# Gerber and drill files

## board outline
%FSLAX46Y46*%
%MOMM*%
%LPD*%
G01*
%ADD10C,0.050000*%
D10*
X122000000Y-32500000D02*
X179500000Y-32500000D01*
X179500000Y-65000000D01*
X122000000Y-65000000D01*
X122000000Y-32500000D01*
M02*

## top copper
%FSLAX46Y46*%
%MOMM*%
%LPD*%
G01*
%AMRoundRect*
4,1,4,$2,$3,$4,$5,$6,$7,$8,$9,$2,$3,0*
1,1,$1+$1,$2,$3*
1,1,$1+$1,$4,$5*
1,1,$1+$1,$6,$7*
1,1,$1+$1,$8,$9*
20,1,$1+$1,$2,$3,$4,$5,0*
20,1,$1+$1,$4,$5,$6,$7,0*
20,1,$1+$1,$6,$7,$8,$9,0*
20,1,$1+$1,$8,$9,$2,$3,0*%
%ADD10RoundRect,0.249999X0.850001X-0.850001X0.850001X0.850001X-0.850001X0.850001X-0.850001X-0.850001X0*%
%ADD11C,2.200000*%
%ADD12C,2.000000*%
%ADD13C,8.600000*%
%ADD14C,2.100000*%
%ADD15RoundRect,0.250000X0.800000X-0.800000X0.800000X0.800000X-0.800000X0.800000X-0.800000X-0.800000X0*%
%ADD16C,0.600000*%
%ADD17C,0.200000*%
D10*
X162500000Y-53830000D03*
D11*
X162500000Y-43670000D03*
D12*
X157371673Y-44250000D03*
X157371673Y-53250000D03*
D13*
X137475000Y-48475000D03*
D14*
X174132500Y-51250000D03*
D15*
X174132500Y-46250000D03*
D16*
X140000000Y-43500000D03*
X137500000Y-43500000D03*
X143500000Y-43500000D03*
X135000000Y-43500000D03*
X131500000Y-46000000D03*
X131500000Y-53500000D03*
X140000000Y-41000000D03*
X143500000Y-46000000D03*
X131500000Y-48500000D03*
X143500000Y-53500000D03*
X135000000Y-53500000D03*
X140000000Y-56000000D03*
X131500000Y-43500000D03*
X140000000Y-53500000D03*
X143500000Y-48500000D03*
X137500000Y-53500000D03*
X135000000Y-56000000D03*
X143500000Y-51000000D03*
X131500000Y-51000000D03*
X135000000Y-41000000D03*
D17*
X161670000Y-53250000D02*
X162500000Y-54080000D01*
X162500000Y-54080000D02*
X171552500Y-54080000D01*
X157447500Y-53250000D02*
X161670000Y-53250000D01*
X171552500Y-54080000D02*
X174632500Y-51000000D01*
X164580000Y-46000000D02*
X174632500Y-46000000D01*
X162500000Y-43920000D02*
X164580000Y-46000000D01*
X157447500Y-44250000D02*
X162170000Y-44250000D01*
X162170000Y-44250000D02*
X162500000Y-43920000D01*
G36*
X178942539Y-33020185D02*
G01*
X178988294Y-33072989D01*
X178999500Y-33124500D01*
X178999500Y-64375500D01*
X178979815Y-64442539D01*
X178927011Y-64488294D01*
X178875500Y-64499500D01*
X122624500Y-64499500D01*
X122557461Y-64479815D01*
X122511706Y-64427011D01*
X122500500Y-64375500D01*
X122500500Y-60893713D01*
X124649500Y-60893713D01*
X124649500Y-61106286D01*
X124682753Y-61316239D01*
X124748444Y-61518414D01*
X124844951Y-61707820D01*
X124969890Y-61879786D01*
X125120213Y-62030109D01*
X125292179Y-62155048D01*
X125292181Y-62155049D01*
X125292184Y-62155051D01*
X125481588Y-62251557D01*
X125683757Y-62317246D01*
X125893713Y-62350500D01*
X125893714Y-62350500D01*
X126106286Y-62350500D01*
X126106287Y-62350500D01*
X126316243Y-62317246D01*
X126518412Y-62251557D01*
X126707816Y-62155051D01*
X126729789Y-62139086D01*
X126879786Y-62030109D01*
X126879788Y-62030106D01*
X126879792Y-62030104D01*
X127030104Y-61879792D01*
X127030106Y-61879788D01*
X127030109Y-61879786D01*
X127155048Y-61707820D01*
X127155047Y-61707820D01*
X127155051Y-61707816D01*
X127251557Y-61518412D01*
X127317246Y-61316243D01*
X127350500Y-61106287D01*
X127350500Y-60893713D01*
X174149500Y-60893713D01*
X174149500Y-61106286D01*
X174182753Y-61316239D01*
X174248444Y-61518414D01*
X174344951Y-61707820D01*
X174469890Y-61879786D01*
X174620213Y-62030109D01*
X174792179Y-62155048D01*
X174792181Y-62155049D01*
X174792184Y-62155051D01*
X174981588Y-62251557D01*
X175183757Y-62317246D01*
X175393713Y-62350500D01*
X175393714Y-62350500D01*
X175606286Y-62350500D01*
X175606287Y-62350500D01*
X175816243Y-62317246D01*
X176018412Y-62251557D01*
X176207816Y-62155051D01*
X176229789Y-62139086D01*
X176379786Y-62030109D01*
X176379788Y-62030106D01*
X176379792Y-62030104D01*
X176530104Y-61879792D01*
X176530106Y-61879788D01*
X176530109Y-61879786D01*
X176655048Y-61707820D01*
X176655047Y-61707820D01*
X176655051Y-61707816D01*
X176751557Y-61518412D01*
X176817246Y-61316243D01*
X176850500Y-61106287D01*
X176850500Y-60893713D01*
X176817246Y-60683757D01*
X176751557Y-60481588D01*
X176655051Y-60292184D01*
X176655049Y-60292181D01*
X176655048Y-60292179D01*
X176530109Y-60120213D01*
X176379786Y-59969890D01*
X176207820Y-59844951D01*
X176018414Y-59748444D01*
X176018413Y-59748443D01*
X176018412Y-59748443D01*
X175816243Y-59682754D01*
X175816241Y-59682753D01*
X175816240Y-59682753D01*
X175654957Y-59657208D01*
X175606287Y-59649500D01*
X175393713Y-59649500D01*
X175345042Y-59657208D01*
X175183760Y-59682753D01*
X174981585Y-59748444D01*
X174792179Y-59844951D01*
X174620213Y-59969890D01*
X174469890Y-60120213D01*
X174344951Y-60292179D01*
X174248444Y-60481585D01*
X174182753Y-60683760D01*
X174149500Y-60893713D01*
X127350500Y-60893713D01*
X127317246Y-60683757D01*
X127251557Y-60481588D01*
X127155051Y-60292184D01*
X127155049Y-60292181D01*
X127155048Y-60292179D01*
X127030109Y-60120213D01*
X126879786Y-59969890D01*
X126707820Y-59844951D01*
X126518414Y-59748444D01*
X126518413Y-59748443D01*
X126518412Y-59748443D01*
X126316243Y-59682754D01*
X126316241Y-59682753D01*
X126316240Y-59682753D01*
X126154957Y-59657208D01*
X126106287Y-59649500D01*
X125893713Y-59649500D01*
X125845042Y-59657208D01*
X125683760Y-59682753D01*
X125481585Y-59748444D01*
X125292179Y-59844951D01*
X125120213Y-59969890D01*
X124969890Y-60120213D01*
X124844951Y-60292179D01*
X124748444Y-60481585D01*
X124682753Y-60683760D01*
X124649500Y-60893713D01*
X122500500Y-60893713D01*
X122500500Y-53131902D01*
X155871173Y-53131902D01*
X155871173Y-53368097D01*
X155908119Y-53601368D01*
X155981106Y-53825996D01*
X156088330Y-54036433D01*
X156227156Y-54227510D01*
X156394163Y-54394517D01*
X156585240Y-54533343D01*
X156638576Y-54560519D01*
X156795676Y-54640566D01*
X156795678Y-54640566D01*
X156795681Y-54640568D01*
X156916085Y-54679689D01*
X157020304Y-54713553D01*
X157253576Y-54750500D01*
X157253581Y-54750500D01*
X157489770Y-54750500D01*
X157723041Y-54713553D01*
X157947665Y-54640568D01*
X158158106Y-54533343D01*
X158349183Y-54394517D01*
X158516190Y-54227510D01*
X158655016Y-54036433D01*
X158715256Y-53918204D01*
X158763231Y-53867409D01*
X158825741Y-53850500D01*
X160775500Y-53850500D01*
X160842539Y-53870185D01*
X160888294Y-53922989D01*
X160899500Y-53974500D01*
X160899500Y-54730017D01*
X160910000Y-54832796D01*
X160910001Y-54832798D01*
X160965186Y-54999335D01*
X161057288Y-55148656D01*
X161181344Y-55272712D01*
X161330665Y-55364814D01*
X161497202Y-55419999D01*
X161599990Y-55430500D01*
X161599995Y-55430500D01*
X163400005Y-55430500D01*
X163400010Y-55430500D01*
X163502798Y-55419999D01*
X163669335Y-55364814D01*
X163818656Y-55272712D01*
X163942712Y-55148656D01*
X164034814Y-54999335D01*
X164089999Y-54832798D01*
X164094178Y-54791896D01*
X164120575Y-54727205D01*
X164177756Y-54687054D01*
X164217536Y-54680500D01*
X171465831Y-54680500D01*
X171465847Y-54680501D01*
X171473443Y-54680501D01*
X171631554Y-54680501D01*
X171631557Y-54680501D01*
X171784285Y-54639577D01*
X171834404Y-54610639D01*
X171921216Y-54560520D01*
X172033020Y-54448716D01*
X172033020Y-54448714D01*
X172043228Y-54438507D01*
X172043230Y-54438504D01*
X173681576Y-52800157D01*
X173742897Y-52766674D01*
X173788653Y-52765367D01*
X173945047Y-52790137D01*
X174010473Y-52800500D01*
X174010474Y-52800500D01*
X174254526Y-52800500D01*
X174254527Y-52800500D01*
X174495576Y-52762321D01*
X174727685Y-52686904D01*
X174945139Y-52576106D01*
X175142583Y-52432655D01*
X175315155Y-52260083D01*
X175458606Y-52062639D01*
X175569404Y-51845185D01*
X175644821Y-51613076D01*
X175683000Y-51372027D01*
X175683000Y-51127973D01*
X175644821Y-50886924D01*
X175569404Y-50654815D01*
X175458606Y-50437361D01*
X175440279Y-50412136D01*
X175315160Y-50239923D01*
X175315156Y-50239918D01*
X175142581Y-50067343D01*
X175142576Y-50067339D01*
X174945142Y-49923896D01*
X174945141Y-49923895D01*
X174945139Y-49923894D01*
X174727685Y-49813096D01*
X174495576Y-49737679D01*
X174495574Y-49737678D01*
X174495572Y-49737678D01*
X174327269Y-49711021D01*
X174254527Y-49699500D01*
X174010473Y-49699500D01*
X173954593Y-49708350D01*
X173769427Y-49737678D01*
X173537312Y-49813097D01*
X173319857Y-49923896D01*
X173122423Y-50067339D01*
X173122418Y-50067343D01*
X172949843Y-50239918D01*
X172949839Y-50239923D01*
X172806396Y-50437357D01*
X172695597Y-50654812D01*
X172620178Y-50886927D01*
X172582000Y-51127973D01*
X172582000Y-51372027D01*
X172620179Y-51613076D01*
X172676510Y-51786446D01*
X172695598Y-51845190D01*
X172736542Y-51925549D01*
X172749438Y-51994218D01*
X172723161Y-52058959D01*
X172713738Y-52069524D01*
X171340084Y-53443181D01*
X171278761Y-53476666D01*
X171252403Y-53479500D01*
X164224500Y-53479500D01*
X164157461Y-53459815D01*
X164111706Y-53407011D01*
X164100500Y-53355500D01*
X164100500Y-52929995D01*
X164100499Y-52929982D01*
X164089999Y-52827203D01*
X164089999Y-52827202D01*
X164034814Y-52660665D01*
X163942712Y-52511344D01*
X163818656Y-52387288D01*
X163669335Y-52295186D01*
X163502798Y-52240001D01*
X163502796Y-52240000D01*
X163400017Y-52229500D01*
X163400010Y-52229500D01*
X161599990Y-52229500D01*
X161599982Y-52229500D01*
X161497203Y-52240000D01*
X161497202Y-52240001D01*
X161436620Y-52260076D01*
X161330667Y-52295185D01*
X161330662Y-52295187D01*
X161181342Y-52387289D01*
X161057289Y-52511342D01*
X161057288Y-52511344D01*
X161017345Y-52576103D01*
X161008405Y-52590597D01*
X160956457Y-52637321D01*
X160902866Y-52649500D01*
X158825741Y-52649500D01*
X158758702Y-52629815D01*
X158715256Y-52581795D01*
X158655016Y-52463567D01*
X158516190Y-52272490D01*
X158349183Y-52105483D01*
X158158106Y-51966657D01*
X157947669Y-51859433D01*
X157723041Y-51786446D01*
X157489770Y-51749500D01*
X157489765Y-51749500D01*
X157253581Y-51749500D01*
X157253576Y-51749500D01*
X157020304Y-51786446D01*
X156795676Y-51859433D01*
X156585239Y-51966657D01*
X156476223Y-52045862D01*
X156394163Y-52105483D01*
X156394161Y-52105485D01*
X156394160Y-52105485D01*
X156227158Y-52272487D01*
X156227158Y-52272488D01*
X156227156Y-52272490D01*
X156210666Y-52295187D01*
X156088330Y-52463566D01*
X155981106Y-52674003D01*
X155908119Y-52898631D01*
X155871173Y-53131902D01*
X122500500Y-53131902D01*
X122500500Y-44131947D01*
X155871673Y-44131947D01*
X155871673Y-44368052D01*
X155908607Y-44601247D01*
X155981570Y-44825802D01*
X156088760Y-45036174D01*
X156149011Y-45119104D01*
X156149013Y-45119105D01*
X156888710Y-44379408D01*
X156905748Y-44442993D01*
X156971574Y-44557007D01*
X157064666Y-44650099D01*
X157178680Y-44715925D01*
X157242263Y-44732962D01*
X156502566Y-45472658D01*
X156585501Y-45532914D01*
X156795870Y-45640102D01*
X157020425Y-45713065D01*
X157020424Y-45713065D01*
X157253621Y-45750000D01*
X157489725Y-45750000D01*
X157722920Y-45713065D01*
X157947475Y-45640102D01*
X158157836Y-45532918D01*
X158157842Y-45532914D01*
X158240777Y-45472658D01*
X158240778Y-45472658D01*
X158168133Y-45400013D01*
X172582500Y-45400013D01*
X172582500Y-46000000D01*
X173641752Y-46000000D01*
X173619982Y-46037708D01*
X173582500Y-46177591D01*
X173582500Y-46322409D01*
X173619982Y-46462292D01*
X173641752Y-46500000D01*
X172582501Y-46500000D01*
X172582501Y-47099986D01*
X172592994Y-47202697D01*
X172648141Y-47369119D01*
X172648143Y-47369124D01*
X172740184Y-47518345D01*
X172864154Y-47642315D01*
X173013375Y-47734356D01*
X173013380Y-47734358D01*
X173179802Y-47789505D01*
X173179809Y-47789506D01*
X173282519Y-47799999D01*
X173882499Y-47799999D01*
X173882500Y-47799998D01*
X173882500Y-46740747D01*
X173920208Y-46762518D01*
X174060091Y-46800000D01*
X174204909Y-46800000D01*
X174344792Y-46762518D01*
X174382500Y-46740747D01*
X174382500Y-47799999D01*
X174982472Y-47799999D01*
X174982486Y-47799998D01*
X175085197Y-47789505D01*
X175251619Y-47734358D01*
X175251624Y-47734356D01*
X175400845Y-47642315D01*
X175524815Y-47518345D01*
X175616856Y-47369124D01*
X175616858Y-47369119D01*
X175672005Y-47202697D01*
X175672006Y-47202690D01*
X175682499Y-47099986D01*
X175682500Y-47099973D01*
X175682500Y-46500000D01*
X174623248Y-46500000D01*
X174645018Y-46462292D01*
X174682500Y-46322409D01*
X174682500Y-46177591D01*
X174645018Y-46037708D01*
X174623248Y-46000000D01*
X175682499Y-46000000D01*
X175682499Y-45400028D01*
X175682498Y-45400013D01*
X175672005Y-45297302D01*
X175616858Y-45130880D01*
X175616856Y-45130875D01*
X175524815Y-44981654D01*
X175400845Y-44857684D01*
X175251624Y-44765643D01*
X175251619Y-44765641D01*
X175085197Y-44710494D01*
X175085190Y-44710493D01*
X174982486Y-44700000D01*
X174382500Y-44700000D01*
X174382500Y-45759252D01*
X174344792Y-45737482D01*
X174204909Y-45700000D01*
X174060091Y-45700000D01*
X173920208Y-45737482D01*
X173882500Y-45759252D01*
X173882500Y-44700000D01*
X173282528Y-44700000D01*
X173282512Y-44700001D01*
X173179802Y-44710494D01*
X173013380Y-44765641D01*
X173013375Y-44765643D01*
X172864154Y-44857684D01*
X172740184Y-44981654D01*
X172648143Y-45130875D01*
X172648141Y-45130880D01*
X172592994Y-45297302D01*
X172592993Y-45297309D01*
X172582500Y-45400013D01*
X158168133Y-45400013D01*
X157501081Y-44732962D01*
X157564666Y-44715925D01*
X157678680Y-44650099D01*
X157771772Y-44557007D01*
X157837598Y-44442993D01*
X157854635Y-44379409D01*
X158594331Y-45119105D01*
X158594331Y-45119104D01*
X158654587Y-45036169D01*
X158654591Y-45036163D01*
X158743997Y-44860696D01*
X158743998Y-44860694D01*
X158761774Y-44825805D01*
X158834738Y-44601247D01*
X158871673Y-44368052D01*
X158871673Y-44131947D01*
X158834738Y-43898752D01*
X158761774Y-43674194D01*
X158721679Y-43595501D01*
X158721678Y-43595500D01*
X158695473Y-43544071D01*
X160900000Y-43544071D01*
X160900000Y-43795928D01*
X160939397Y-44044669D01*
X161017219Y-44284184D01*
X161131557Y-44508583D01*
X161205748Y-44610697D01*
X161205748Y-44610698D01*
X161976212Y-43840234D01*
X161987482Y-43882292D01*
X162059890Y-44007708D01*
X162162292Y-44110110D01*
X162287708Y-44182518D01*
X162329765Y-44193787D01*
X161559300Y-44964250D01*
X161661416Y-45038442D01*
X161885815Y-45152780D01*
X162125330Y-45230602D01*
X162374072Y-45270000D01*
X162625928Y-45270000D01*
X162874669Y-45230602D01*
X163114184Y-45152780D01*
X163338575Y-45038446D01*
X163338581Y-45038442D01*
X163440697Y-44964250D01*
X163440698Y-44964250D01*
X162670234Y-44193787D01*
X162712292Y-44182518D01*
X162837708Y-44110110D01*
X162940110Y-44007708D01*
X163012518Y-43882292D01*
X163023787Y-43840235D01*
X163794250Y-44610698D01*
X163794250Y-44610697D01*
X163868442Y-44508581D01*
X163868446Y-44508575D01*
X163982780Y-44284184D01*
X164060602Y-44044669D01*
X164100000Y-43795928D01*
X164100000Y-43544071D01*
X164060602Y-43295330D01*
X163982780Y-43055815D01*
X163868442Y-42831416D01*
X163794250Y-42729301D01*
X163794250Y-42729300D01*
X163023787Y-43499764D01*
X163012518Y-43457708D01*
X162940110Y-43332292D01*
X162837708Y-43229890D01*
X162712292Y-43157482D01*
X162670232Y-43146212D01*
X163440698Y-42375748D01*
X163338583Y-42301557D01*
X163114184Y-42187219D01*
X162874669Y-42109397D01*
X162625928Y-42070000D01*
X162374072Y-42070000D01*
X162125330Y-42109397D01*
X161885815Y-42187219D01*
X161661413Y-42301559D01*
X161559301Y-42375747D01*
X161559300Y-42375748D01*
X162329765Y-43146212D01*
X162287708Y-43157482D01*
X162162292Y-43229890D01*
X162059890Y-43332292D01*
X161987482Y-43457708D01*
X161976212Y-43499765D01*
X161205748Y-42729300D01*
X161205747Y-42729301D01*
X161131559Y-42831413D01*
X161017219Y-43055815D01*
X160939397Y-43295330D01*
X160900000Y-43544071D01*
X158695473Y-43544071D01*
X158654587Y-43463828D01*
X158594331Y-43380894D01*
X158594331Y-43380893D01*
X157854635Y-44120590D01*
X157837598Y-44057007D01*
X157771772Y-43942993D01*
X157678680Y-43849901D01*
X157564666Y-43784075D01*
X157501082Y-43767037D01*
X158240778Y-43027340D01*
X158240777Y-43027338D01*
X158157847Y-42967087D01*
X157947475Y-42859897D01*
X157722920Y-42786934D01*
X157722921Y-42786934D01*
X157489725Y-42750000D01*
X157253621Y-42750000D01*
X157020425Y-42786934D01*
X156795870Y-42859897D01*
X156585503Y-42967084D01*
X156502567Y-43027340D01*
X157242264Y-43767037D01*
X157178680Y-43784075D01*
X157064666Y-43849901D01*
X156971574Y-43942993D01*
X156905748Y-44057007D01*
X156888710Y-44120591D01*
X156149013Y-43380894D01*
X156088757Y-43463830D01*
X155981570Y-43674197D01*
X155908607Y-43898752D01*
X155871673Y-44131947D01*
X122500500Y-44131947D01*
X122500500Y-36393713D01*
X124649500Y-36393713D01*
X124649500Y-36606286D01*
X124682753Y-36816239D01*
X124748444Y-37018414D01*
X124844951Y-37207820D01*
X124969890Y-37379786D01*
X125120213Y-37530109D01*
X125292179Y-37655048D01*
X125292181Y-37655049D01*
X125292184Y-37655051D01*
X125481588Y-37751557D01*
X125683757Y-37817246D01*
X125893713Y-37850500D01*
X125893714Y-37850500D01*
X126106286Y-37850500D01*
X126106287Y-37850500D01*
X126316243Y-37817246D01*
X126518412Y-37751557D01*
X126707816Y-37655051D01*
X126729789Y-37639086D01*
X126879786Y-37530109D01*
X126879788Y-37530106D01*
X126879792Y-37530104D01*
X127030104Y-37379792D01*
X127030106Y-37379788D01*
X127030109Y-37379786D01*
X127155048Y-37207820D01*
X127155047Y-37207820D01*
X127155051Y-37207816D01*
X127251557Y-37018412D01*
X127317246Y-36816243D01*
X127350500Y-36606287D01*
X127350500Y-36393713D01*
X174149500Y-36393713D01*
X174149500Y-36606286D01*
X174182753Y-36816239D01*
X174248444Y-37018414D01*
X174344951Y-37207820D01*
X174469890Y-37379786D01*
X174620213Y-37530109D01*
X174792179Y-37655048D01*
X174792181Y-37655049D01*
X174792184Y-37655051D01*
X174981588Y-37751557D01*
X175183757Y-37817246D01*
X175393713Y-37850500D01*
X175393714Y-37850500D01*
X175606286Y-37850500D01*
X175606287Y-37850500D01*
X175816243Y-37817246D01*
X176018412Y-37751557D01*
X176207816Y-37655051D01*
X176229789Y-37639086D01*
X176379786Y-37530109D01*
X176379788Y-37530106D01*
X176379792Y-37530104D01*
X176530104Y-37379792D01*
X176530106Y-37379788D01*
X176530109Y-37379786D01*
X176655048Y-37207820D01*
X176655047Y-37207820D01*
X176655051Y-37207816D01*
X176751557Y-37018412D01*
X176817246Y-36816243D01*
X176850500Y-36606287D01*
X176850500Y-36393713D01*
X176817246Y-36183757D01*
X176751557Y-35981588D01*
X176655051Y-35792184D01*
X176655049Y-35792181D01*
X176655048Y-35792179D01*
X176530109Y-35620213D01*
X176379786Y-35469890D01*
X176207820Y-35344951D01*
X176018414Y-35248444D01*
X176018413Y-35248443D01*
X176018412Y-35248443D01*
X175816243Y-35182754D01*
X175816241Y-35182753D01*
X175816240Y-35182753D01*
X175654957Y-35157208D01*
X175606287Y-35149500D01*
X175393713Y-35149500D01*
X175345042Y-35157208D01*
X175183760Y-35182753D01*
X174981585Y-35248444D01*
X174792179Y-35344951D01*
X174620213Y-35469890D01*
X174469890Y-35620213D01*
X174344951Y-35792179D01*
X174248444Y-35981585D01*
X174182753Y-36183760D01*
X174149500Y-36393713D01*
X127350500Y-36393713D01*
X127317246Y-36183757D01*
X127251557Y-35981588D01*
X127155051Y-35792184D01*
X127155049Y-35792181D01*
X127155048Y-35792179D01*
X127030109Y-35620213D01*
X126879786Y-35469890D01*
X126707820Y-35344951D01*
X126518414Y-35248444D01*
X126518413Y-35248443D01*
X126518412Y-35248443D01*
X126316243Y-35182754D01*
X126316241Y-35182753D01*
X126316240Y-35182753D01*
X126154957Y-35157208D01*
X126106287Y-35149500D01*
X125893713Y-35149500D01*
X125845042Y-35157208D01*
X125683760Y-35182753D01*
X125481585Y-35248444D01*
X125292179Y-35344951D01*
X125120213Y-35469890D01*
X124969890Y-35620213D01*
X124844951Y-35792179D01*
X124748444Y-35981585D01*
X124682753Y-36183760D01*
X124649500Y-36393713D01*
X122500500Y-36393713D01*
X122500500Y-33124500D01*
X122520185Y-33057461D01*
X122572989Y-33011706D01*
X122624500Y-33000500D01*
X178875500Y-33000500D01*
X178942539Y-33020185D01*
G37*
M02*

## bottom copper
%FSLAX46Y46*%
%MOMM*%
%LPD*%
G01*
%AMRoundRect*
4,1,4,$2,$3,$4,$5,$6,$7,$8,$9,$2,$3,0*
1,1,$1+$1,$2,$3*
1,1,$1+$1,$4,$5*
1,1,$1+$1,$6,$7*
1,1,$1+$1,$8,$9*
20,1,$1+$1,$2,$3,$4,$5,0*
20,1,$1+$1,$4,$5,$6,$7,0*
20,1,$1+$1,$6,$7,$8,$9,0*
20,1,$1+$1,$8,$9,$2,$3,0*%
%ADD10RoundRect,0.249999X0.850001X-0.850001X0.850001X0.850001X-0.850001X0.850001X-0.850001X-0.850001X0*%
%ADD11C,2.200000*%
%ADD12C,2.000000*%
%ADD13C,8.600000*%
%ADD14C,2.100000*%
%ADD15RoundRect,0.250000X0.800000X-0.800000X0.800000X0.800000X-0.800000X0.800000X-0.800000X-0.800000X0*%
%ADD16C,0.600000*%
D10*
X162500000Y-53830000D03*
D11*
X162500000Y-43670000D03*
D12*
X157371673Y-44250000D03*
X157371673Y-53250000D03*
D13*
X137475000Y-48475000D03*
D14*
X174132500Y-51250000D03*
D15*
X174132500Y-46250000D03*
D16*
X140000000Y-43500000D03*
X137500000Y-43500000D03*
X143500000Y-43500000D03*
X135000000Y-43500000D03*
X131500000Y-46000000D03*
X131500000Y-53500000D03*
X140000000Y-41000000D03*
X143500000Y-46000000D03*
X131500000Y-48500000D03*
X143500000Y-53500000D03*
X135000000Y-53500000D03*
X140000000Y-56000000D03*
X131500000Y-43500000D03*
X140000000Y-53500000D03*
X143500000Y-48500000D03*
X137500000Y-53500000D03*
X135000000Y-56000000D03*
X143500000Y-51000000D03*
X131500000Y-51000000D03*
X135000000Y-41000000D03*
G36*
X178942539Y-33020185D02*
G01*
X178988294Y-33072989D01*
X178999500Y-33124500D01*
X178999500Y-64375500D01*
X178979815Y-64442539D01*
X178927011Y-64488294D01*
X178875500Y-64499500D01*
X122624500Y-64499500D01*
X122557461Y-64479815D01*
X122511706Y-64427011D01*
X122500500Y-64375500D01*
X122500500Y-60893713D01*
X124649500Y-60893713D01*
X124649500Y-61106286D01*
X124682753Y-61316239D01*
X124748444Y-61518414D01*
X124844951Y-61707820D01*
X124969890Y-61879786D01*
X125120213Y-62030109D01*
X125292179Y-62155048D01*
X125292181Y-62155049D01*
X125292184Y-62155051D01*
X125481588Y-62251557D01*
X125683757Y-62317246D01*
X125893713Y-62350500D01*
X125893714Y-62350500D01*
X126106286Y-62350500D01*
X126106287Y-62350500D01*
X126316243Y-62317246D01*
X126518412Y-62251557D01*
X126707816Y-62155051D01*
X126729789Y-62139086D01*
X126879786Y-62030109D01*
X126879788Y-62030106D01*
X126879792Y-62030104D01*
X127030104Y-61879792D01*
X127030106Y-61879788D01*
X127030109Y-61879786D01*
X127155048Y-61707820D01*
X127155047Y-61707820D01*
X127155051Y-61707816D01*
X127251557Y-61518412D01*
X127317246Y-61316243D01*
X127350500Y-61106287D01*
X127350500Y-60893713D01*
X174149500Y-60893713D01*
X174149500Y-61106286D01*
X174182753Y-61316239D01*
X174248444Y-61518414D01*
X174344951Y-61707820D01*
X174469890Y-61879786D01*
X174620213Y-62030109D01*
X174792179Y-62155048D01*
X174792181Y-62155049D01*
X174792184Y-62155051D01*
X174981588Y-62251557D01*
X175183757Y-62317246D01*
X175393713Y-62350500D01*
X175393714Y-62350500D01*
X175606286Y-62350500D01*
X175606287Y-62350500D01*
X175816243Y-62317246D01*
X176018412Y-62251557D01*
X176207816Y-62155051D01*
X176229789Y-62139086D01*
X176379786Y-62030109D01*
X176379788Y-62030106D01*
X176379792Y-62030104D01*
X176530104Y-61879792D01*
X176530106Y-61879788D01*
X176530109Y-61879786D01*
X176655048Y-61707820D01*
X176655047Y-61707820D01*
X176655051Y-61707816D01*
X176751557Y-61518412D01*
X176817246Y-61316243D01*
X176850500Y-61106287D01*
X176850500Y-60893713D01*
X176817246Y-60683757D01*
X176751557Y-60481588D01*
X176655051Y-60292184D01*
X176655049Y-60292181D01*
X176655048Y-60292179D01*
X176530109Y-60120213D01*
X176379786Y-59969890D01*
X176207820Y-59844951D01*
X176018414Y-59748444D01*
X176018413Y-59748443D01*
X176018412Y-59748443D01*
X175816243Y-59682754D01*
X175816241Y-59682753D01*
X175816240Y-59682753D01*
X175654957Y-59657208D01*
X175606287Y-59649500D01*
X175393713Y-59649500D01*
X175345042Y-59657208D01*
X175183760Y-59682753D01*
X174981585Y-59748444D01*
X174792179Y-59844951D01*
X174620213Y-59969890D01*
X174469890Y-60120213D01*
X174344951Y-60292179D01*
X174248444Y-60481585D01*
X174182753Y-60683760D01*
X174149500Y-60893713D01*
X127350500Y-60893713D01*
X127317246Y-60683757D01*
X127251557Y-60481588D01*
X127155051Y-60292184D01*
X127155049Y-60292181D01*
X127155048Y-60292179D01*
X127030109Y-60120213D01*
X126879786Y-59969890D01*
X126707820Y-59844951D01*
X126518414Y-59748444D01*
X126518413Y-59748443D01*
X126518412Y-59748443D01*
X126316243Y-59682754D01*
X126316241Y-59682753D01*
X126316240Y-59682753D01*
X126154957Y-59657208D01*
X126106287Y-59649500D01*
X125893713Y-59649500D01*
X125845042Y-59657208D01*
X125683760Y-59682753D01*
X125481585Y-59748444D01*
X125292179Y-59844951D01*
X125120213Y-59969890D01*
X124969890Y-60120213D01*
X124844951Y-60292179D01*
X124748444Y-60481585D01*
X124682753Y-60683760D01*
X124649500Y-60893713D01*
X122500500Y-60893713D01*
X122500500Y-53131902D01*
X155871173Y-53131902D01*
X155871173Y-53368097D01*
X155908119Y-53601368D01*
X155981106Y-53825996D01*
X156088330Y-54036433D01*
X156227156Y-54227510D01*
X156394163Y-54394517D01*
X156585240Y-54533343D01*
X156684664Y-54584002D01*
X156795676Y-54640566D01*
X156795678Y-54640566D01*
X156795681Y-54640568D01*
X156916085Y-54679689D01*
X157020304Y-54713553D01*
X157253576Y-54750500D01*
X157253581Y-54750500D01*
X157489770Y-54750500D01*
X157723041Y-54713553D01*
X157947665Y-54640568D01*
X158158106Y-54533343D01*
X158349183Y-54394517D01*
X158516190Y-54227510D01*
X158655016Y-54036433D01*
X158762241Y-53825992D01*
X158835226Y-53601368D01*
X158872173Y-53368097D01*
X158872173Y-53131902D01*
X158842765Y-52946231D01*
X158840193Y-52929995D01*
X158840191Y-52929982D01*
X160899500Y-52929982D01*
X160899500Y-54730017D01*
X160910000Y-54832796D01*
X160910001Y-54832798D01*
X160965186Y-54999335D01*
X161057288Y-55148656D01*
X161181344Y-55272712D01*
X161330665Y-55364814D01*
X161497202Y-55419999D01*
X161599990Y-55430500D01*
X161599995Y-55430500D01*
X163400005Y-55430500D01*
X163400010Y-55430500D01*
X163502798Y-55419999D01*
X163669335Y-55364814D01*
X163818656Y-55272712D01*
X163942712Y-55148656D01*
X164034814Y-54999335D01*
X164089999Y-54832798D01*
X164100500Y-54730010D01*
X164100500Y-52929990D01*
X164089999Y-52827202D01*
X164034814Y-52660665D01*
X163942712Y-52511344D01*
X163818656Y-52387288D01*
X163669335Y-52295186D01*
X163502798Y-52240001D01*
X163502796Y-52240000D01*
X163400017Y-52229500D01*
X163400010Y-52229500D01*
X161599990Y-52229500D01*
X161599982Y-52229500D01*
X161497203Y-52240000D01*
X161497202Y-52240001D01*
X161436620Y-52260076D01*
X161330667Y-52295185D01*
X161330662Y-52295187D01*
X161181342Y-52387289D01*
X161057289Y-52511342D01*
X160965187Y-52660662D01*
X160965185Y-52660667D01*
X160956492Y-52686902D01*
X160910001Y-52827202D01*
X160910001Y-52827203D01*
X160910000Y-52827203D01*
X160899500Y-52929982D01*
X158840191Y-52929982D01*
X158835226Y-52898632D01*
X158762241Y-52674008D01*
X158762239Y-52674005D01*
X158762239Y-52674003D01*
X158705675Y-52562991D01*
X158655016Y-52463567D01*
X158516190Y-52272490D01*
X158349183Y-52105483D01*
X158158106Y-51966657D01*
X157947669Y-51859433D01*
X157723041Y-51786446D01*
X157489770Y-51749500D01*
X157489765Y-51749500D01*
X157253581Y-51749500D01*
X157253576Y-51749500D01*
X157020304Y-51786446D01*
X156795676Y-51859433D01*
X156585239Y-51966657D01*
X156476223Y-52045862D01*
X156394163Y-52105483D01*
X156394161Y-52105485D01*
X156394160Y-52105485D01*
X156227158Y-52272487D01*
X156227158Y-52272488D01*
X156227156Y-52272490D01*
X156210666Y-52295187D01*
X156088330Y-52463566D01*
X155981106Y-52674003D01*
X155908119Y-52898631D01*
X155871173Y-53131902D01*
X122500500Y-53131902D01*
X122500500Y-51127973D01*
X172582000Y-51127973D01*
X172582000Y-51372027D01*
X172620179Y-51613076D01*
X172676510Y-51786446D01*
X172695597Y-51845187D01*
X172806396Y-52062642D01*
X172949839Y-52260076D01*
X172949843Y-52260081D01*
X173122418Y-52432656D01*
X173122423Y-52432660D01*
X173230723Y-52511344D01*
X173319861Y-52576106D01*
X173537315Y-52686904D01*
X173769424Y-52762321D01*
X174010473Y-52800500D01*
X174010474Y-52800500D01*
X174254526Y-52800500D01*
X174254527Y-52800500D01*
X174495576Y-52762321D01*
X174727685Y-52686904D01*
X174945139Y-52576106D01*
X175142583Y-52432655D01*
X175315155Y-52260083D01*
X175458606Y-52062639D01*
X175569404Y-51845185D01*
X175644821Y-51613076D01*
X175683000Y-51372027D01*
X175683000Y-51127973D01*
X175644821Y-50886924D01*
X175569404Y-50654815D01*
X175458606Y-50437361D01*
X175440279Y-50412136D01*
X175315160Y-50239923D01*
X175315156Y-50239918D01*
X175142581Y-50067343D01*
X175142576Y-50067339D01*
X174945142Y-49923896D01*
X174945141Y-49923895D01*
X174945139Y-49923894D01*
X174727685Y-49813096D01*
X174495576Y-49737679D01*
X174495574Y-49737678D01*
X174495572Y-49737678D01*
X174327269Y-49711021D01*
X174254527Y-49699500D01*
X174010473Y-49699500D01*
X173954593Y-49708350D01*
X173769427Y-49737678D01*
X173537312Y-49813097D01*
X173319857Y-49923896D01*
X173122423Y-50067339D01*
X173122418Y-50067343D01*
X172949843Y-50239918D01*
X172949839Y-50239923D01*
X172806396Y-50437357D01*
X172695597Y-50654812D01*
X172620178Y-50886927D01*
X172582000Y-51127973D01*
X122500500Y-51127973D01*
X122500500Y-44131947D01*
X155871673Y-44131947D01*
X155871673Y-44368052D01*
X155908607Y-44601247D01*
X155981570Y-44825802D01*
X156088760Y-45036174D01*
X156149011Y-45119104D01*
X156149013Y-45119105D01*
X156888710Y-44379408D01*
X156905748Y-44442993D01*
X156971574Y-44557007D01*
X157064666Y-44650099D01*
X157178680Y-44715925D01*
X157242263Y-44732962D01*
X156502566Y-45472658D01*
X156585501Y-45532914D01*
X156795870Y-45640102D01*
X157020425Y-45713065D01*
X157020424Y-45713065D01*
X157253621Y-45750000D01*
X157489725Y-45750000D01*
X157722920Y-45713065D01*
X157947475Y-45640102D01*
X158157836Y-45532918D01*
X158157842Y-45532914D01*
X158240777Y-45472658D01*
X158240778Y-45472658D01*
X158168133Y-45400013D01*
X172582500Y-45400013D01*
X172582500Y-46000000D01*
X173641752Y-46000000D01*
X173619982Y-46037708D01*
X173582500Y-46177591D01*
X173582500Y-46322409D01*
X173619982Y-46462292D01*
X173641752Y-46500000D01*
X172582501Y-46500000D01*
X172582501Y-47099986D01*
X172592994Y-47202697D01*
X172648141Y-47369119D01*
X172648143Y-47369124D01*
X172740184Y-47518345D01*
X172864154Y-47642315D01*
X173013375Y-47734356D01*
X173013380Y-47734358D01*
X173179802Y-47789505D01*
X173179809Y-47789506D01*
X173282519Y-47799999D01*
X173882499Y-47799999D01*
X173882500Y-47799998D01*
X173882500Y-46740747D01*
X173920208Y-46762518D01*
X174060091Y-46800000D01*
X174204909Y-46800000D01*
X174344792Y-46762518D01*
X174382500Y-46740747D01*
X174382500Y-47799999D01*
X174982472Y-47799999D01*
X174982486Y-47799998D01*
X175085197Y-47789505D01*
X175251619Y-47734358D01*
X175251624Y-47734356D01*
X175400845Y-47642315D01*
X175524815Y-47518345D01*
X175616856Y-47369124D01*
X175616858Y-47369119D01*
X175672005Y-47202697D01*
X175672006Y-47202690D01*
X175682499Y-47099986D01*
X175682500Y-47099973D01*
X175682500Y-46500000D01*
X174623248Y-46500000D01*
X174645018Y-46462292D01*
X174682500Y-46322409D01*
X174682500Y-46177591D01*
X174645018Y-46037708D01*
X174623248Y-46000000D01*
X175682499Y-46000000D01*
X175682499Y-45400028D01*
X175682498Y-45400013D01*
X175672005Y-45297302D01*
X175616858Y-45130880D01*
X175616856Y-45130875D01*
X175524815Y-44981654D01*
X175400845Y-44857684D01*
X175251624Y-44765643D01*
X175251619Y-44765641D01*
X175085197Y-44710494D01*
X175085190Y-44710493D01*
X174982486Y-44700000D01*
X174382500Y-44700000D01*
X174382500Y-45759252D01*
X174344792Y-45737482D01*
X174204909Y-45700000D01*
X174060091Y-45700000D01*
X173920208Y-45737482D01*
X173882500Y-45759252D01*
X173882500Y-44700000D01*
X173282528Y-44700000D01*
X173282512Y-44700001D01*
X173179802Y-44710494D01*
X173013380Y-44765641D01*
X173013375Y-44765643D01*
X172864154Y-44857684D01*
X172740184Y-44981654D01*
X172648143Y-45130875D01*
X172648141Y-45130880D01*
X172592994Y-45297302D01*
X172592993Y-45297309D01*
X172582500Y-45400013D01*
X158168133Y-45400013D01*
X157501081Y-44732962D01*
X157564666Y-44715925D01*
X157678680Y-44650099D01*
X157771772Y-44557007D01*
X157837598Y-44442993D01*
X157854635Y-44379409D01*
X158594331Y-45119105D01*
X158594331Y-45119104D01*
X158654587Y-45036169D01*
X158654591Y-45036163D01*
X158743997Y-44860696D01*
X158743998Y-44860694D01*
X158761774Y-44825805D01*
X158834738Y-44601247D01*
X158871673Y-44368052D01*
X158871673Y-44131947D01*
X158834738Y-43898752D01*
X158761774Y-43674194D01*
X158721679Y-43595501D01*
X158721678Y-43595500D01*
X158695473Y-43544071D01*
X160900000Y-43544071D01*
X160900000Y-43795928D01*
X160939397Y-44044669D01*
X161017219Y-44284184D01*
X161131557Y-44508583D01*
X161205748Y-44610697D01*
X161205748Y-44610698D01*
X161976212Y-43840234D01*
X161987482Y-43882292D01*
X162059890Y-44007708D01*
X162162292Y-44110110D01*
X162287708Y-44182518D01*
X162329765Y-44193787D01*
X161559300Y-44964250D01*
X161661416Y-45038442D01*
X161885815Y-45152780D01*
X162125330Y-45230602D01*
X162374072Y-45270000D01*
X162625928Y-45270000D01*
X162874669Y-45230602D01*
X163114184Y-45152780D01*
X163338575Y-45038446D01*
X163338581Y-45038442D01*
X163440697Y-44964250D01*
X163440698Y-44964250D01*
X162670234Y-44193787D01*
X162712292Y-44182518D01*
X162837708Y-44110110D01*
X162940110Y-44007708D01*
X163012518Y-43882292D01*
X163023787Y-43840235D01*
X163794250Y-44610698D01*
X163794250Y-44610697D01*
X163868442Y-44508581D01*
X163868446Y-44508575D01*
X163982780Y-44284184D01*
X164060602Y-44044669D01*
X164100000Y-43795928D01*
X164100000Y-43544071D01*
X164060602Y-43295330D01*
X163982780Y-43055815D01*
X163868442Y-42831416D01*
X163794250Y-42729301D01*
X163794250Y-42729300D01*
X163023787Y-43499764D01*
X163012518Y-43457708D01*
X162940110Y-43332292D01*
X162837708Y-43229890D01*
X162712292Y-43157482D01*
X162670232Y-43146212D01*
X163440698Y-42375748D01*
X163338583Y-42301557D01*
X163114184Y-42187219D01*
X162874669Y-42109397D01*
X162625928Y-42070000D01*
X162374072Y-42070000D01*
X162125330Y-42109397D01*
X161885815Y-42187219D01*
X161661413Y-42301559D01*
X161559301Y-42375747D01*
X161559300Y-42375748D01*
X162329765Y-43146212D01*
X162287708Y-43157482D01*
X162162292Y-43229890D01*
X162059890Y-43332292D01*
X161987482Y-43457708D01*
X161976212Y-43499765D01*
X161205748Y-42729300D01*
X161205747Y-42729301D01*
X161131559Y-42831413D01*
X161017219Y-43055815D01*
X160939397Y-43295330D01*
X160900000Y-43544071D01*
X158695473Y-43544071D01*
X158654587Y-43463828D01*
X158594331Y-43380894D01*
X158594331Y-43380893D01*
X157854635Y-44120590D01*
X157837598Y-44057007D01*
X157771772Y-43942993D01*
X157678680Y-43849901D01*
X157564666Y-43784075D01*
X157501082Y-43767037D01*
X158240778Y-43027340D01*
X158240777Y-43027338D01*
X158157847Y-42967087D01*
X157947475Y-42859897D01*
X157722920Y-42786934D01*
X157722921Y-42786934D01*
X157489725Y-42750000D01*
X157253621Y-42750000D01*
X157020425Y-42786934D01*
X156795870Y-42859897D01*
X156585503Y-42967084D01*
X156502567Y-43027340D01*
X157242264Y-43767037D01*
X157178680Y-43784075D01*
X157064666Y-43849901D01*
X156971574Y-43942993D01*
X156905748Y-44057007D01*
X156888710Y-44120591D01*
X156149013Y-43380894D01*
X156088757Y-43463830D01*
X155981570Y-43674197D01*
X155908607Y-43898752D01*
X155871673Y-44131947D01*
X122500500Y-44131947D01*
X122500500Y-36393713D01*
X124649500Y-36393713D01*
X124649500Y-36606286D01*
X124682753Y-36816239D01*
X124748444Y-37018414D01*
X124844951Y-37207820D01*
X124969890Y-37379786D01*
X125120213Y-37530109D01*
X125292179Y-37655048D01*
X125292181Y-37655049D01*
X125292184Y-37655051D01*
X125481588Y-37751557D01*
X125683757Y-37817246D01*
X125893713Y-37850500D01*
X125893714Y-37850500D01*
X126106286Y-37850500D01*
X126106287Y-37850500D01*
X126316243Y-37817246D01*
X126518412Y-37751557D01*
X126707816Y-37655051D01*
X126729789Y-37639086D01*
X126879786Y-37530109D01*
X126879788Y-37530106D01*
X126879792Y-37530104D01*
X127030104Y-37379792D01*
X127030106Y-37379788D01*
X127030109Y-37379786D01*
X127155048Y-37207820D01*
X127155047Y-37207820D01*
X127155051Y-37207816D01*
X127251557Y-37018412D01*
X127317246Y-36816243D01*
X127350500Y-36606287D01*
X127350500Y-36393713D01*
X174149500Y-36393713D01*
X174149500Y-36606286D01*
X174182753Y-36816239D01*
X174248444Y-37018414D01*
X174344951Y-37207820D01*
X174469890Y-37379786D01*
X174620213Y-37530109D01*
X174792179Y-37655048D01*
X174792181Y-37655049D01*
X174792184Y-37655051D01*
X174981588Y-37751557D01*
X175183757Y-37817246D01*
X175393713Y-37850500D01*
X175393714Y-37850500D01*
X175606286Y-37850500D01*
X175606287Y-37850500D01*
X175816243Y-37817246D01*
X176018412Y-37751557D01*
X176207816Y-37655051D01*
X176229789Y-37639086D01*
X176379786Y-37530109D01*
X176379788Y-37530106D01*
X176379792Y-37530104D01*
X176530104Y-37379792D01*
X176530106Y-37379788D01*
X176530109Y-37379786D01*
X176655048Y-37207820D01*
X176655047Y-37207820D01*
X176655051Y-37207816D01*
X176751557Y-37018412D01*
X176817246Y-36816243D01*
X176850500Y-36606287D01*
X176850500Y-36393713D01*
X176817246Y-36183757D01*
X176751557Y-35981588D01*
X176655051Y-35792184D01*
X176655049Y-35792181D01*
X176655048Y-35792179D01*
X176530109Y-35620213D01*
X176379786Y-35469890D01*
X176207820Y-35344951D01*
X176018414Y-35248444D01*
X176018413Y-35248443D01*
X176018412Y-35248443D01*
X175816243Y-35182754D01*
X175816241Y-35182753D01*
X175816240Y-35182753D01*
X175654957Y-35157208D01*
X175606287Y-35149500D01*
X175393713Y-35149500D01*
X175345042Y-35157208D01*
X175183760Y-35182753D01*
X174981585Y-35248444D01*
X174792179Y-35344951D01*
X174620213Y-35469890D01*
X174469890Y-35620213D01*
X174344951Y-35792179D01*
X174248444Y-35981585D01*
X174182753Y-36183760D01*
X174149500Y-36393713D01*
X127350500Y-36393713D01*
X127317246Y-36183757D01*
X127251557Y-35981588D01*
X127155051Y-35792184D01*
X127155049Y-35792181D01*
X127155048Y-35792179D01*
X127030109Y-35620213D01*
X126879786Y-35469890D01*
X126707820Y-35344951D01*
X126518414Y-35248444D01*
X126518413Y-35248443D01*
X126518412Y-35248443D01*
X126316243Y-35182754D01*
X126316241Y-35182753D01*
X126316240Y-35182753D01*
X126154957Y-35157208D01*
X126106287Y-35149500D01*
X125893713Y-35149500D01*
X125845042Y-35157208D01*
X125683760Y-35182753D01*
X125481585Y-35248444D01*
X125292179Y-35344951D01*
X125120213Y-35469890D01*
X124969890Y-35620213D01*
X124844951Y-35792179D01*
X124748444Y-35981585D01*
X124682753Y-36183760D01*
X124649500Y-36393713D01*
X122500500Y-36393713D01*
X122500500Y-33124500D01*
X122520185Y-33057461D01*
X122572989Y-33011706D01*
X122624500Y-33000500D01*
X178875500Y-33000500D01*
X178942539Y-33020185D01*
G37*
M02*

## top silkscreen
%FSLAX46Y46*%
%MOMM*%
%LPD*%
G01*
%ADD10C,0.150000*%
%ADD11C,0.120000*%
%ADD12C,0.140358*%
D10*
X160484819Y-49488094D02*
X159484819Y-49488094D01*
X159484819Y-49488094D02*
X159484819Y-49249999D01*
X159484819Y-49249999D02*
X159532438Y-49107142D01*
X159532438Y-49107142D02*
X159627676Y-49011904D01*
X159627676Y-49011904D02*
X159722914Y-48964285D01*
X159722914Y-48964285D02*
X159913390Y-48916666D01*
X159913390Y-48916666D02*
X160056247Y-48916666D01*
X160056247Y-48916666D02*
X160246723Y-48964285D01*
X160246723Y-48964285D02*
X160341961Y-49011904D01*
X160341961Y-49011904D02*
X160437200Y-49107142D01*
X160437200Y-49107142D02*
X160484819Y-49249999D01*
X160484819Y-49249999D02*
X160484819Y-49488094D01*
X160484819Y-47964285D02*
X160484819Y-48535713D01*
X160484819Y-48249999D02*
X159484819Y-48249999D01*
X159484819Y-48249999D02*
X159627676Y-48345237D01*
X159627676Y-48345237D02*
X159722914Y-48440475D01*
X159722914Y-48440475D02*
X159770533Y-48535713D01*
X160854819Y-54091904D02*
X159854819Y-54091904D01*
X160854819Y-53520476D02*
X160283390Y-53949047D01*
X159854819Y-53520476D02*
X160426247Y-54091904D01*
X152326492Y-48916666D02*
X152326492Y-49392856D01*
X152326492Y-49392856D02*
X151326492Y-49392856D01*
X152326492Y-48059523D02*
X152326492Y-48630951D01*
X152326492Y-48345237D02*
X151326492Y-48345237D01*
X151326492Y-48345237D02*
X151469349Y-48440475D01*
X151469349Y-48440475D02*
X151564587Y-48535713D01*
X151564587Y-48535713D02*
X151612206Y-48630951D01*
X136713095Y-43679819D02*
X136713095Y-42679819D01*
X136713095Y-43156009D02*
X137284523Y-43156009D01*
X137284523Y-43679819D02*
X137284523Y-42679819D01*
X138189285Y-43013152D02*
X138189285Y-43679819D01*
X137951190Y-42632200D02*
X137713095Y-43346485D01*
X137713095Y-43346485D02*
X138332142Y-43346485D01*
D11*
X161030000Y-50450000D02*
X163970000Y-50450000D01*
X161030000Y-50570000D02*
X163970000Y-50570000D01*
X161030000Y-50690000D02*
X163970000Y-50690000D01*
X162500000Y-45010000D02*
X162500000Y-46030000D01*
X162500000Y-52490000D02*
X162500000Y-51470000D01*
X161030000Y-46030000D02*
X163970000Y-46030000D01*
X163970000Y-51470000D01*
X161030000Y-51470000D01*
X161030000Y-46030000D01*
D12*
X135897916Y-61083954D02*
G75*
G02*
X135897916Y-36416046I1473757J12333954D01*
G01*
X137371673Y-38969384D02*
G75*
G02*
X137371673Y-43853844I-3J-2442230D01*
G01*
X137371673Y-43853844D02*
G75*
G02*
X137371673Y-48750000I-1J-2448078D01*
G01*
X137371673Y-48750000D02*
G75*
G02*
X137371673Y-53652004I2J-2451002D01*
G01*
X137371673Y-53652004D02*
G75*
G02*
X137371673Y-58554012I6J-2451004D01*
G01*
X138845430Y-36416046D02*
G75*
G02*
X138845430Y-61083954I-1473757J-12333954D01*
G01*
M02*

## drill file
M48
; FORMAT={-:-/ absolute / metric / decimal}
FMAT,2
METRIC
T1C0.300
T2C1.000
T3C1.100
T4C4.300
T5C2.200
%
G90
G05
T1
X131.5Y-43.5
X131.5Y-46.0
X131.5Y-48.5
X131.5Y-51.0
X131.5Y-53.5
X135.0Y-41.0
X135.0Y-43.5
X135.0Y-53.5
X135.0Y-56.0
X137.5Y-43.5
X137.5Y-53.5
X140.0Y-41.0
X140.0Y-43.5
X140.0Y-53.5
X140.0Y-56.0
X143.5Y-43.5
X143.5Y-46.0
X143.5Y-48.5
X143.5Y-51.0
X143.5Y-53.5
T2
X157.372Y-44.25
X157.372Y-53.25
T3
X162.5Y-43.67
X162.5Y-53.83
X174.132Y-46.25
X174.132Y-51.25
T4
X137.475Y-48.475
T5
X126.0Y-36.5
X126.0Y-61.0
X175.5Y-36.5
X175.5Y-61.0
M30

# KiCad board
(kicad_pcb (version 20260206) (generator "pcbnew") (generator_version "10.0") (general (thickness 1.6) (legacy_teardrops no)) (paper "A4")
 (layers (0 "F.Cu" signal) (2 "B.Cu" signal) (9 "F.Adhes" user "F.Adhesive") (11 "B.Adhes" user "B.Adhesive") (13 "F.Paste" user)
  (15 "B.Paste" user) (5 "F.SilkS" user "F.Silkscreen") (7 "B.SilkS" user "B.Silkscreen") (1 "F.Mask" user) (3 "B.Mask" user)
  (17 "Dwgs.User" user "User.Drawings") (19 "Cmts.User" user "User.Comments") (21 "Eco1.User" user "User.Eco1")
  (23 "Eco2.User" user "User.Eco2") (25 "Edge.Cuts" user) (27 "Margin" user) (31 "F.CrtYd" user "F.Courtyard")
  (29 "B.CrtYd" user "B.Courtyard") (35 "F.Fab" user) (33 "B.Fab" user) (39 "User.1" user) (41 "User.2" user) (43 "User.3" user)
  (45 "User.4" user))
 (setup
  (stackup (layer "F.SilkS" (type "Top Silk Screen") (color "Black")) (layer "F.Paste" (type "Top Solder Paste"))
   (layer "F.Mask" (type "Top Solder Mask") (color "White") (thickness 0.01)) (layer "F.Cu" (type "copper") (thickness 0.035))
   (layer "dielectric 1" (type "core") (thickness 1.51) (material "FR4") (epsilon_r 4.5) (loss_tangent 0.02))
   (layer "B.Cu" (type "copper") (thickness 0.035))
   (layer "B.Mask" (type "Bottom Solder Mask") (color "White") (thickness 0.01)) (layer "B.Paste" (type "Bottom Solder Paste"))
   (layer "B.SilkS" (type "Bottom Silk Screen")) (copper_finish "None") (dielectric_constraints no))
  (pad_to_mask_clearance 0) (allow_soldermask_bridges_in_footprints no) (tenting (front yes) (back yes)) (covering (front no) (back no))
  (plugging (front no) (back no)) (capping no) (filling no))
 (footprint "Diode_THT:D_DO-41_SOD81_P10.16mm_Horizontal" (layer "F.Cu") (at 162.5 53.83 90)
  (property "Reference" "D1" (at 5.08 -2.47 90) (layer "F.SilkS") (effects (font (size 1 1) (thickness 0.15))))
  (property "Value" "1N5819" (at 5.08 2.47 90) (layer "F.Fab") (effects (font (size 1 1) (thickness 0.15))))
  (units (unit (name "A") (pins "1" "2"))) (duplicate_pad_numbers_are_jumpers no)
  (fp_line (start 3.38 -1.47) (end 3.38 1.47) (stroke (width 0.12) (type solid)) (layer "F.SilkS"))
  (fp_line (start 3.26 -1.47) (end 3.26 1.47) (stroke (width 0.12) (type solid)) (layer "F.SilkS"))
  (fp_line (start 3.14 -1.47) (end 3.14 1.47) (stroke (width 0.12) (type solid)) (layer "F.SilkS"))
  (fp_line (start 8.82 0) (end 7.8 0) (stroke (width 0.12) (type solid)) (layer "F.SilkS"))
  (fp_line (start 1.34 0) (end 2.36 0) (stroke (width 0.12) (type solid)) (layer "F.SilkS"))
  (fp_rect (start 2.36 -1.47) (end 7.8 1.47) (stroke (width 0.12) (type solid)) (fill no) (layer "F.SilkS"))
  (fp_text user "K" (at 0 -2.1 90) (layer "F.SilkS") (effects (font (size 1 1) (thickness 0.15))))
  (pad "1" thru_hole roundrect (at 0 0 90) (size 2.2 2.2) (drill 1.1) (layers "*.Cu" "*.Mask") (remove_unused_layers no)
   (roundrect_rratio 0.113636) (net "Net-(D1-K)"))
  (pad "2" thru_hole circle (at 10.16 0 90) (size 2.2 2.2) (drill 1.1) (layers "*.Cu" "*.Mask") (remove_unused_layers no) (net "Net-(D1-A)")))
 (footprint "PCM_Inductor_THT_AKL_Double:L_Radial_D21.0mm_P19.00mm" (layer "F.Cu") (at 137.371673 36.25 -90)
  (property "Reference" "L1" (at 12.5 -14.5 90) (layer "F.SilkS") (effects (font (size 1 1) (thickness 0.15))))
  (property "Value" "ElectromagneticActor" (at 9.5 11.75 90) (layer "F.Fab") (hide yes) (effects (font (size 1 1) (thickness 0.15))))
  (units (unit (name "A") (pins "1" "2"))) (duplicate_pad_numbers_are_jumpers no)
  (fp_arc (start 24.833954 1.473757) (mid 12.5 12.42169) (end 0.166046 1.473757) (stroke (width 0.140358) (type solid)) (layer "F.SilkS"))
  (fp_arc (start 2.719384 0) (mid 5.161611 -2.442227) (end 7.603844 0) (stroke (width 0.140358) (type solid)) (layer "F.SilkS"))
  (fp_arc (start 7.603844 0) (mid 10.051921 -2.448077) (end 12.5 0) (stroke (width 0.140358) (type solid)) (layer "F.SilkS"))
  (fp_arc (start 12.5 0) (mid 14.951004 -2.451004) (end 17.402004 0) (stroke (width 0.140358) (type solid)) (layer "F.SilkS"))
  (fp_arc (start 17.402004 0) (mid 19.853013 -2.451009) (end 22.304011 0) (stroke (width 0.140358) (type solid)) (layer "F.SilkS"))
  (fp_arc (start 0.166046 -1.473757) (mid 12.5 -12.42169) (end 24.833954 -1.473757) (stroke (width 0.140358) (type solid)) (layer "F.SilkS"))
  (pad "1" thru_hole circle (at 8 -20 270) (size 2 2) (drill 1) (layers "*.Cu" "*.Mask") (remove_unused_layers no) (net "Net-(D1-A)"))
  (pad "2" thru_hole circle (at 17 -20 270) (size 2 2) (drill 1) (layers "*.Cu" "*.Mask") (remove_unused_layers no) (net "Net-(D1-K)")))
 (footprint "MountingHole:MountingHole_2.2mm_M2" (layer "F.Cu") (at 126 61)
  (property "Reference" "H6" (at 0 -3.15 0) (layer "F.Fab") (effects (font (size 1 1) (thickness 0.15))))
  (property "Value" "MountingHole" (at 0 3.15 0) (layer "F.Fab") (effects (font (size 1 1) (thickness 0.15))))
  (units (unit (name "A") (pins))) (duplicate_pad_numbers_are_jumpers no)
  (pad "" np_thru_hole circle (at 0 0) (size 2.2 2.2) (drill 2.2) (layers "*.Cu" "*.Mask")))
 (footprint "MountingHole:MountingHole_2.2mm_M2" (layer "F.Cu") (at 175.5 61)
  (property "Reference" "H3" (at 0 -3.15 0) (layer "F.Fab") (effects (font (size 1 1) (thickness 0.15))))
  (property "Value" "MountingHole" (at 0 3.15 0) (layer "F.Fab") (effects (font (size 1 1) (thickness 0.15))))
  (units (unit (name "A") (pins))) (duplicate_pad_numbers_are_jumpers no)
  (pad "" np_thru_hole circle (at 0 0) (size 2.2 2.2) (drill 2.2) (layers "*.Cu" "*.Mask")))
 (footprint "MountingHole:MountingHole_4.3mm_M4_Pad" (layer "F.Cu") (at 137.475 48.475)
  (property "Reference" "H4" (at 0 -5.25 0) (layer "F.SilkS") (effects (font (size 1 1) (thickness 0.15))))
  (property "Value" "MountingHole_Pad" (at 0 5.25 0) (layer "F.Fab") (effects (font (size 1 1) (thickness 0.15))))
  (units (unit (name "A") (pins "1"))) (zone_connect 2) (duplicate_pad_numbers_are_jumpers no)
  (pad "1" thru_hole circle (at 0 0) (size 8.6 8.6) (drill 4.3) (layers "*.Cu" "*.Mask") (remove_unused_layers no) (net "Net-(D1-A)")
   (zone_connect 2)))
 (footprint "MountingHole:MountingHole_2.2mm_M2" (layer "F.Cu") (at 126 36.5)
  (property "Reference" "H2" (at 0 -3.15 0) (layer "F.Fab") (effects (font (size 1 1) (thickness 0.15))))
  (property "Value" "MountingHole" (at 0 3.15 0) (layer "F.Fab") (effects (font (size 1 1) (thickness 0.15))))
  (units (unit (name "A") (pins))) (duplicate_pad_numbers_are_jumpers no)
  (pad "" np_thru_hole circle (at 0 0) (size 2.2 2.2) (drill 2.2) (layers "*.Cu" "*.Mask")))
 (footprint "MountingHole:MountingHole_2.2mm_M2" (layer "F.Cu") (at 175.5 36.5)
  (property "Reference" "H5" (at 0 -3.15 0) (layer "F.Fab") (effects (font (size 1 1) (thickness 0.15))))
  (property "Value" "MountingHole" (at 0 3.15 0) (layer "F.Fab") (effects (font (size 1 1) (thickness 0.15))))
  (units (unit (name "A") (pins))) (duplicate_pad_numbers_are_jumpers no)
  (pad "" np_thru_hole circle (at 0 0) (size 2.2 2.2) (drill 2.2) (layers "*.Cu" "*.Mask")))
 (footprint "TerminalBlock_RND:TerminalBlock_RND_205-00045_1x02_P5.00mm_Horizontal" (layer "B.Cu") (at 174.1325 51.25 90)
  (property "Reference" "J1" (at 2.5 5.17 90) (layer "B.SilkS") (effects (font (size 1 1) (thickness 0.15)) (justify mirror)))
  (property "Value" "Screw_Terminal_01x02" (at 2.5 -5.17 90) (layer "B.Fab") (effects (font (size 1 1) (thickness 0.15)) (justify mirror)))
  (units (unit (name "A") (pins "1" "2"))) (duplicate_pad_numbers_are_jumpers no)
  (pad "1" thru_hole circle (at 0 0 90) (size 2.1 2.1) (drill 1.1) (layers "*.Cu" "*.Mask") (remove_unused_layers no) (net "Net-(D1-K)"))
  (pad "2" thru_hole roundrect (at 5 0 90) (size 2.1 2.1) (drill 1.1) (layers "*.Cu" "*.Mask") (remove_unused_layers no)
   (roundrect_rratio 0.119047619) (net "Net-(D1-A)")))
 (gr_rect (start 122 32.5) (end 179.5 65) (stroke (width 0.05) (type default)) (fill no) (layer "Edge.Cuts"))
 (segment (start 161.67 53.25) (end 162.5 54.08) (width 0.2) (layer "F.Cu") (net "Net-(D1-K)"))
 (segment (start 162.5 54.08) (end 171.5525 54.08) (width 0.2) (layer "F.Cu") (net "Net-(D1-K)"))
 (segment (start 157.4475 53.25) (end 161.67 53.25) (width 0.2) (layer "F.Cu") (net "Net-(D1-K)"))
 (segment (start 171.5525 54.08) (end 174.6325 51) (width 0.2) (layer "F.Cu") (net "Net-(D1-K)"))
 (segment (start 164.58 46) (end 174.6325 46) (width 0.2) (layer "F.Cu") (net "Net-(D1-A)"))
 (segment (start 162.5 43.92) (end 164.58 46) (width 0.2) (layer "F.Cu") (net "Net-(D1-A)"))
 (segment (start 157.4475 44.25) (end 162.17 44.25) (width 0.2) (layer "F.Cu") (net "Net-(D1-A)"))
 (segment (start 162.17 44.25) (end 162.5 43.92) (width 0.2) (layer "F.Cu") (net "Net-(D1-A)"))
 (via (at 140 43.5) (size 0.6) (drill 0.3) (layers "F.Cu" "B.Cu") (free yes) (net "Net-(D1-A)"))
 (via (at 137.5 43.5) (size 0.6) (drill 0.3) (layers "F.Cu" "B.Cu") (free yes) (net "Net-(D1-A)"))
 (via (at 143.5 43.5) (size 0.6) (drill 0.3) (layers "F.Cu" "B.Cu") (free yes) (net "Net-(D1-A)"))
 (via (at 135 43.5) (size 0.6) (drill 0.3) (layers "F.Cu" "B.Cu") (free yes) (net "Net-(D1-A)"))
 (via (at 131.5 46) (size 0.6) (drill 0.3) (layers "F.Cu" "B.Cu") (free yes) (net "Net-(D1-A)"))
 (via (at 131.5 53.5) (size 0.6) (drill 0.3) (layers "F.Cu" "B.Cu") (free yes) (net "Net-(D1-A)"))
 (via (at 140 41) (size 0.6) (drill 0.3) (layers "F.Cu" "B.Cu") (free yes) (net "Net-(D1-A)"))
 (via (at 143.5 46) (size 0.6) (drill 0.3) (layers "F.Cu" "B.Cu") (free yes) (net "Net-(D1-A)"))
 (via (at 131.5 48.5) (size 0.6) (drill 0.3) (layers "F.Cu" "B.Cu") (free yes) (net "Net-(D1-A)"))
 (via (at 143.5 53.5) (size 0.6) (drill 0.3) (layers "F.Cu" "B.Cu") (free yes) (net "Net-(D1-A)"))
 (via (at 135 53.5) (size 0.6) (drill 0.3) (layers "F.Cu" "B.Cu") (free yes) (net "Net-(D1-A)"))
 (via (at 140 56) (size 0.6) (drill 0.3) (layers "F.Cu" "B.Cu") (free yes) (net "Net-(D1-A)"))
 (via (at 131.5 43.5) (size 0.6) (drill 0.3) (layers "F.Cu" "B.Cu") (free yes) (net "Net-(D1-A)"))
 (via (at 140 53.5) (size 0.6) (drill 0.3) (layers "F.Cu" "B.Cu") (free yes) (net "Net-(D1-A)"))
 (via (at 143.5 48.5) (size 0.6) (drill 0.3) (layers "F.Cu" "B.Cu") (free yes) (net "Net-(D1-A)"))
 (via (at 137.5 53.5) (size 0.6) (drill 0.3) (layers "F.Cu" "B.Cu") (free yes) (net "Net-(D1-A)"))
 (via (at 135 56) (size 0.6) (drill 0.3) (layers "F.Cu" "B.Cu") (free yes) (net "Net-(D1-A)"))
 (via (at 143.5 51) (size 0.6) (drill 0.3) (layers "F.Cu" "B.Cu") (free yes) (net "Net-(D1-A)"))
 (via (at 131.5 51) (size 0.6) (drill 0.3) (layers "F.Cu" "B.Cu") (free yes) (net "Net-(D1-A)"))
 (via (at 135 41) (size 0.6) (drill 0.3) (layers "F.Cu" "B.Cu") (free yes) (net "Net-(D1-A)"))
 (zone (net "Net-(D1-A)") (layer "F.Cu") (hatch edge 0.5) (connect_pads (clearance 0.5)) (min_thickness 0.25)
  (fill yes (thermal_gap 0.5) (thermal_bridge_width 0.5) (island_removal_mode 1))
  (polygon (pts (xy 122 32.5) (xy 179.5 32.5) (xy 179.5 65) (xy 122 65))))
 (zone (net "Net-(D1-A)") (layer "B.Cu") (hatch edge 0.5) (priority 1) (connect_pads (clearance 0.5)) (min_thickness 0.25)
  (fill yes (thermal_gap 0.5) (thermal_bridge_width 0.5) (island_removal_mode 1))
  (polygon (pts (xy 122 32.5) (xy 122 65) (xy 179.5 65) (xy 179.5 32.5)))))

